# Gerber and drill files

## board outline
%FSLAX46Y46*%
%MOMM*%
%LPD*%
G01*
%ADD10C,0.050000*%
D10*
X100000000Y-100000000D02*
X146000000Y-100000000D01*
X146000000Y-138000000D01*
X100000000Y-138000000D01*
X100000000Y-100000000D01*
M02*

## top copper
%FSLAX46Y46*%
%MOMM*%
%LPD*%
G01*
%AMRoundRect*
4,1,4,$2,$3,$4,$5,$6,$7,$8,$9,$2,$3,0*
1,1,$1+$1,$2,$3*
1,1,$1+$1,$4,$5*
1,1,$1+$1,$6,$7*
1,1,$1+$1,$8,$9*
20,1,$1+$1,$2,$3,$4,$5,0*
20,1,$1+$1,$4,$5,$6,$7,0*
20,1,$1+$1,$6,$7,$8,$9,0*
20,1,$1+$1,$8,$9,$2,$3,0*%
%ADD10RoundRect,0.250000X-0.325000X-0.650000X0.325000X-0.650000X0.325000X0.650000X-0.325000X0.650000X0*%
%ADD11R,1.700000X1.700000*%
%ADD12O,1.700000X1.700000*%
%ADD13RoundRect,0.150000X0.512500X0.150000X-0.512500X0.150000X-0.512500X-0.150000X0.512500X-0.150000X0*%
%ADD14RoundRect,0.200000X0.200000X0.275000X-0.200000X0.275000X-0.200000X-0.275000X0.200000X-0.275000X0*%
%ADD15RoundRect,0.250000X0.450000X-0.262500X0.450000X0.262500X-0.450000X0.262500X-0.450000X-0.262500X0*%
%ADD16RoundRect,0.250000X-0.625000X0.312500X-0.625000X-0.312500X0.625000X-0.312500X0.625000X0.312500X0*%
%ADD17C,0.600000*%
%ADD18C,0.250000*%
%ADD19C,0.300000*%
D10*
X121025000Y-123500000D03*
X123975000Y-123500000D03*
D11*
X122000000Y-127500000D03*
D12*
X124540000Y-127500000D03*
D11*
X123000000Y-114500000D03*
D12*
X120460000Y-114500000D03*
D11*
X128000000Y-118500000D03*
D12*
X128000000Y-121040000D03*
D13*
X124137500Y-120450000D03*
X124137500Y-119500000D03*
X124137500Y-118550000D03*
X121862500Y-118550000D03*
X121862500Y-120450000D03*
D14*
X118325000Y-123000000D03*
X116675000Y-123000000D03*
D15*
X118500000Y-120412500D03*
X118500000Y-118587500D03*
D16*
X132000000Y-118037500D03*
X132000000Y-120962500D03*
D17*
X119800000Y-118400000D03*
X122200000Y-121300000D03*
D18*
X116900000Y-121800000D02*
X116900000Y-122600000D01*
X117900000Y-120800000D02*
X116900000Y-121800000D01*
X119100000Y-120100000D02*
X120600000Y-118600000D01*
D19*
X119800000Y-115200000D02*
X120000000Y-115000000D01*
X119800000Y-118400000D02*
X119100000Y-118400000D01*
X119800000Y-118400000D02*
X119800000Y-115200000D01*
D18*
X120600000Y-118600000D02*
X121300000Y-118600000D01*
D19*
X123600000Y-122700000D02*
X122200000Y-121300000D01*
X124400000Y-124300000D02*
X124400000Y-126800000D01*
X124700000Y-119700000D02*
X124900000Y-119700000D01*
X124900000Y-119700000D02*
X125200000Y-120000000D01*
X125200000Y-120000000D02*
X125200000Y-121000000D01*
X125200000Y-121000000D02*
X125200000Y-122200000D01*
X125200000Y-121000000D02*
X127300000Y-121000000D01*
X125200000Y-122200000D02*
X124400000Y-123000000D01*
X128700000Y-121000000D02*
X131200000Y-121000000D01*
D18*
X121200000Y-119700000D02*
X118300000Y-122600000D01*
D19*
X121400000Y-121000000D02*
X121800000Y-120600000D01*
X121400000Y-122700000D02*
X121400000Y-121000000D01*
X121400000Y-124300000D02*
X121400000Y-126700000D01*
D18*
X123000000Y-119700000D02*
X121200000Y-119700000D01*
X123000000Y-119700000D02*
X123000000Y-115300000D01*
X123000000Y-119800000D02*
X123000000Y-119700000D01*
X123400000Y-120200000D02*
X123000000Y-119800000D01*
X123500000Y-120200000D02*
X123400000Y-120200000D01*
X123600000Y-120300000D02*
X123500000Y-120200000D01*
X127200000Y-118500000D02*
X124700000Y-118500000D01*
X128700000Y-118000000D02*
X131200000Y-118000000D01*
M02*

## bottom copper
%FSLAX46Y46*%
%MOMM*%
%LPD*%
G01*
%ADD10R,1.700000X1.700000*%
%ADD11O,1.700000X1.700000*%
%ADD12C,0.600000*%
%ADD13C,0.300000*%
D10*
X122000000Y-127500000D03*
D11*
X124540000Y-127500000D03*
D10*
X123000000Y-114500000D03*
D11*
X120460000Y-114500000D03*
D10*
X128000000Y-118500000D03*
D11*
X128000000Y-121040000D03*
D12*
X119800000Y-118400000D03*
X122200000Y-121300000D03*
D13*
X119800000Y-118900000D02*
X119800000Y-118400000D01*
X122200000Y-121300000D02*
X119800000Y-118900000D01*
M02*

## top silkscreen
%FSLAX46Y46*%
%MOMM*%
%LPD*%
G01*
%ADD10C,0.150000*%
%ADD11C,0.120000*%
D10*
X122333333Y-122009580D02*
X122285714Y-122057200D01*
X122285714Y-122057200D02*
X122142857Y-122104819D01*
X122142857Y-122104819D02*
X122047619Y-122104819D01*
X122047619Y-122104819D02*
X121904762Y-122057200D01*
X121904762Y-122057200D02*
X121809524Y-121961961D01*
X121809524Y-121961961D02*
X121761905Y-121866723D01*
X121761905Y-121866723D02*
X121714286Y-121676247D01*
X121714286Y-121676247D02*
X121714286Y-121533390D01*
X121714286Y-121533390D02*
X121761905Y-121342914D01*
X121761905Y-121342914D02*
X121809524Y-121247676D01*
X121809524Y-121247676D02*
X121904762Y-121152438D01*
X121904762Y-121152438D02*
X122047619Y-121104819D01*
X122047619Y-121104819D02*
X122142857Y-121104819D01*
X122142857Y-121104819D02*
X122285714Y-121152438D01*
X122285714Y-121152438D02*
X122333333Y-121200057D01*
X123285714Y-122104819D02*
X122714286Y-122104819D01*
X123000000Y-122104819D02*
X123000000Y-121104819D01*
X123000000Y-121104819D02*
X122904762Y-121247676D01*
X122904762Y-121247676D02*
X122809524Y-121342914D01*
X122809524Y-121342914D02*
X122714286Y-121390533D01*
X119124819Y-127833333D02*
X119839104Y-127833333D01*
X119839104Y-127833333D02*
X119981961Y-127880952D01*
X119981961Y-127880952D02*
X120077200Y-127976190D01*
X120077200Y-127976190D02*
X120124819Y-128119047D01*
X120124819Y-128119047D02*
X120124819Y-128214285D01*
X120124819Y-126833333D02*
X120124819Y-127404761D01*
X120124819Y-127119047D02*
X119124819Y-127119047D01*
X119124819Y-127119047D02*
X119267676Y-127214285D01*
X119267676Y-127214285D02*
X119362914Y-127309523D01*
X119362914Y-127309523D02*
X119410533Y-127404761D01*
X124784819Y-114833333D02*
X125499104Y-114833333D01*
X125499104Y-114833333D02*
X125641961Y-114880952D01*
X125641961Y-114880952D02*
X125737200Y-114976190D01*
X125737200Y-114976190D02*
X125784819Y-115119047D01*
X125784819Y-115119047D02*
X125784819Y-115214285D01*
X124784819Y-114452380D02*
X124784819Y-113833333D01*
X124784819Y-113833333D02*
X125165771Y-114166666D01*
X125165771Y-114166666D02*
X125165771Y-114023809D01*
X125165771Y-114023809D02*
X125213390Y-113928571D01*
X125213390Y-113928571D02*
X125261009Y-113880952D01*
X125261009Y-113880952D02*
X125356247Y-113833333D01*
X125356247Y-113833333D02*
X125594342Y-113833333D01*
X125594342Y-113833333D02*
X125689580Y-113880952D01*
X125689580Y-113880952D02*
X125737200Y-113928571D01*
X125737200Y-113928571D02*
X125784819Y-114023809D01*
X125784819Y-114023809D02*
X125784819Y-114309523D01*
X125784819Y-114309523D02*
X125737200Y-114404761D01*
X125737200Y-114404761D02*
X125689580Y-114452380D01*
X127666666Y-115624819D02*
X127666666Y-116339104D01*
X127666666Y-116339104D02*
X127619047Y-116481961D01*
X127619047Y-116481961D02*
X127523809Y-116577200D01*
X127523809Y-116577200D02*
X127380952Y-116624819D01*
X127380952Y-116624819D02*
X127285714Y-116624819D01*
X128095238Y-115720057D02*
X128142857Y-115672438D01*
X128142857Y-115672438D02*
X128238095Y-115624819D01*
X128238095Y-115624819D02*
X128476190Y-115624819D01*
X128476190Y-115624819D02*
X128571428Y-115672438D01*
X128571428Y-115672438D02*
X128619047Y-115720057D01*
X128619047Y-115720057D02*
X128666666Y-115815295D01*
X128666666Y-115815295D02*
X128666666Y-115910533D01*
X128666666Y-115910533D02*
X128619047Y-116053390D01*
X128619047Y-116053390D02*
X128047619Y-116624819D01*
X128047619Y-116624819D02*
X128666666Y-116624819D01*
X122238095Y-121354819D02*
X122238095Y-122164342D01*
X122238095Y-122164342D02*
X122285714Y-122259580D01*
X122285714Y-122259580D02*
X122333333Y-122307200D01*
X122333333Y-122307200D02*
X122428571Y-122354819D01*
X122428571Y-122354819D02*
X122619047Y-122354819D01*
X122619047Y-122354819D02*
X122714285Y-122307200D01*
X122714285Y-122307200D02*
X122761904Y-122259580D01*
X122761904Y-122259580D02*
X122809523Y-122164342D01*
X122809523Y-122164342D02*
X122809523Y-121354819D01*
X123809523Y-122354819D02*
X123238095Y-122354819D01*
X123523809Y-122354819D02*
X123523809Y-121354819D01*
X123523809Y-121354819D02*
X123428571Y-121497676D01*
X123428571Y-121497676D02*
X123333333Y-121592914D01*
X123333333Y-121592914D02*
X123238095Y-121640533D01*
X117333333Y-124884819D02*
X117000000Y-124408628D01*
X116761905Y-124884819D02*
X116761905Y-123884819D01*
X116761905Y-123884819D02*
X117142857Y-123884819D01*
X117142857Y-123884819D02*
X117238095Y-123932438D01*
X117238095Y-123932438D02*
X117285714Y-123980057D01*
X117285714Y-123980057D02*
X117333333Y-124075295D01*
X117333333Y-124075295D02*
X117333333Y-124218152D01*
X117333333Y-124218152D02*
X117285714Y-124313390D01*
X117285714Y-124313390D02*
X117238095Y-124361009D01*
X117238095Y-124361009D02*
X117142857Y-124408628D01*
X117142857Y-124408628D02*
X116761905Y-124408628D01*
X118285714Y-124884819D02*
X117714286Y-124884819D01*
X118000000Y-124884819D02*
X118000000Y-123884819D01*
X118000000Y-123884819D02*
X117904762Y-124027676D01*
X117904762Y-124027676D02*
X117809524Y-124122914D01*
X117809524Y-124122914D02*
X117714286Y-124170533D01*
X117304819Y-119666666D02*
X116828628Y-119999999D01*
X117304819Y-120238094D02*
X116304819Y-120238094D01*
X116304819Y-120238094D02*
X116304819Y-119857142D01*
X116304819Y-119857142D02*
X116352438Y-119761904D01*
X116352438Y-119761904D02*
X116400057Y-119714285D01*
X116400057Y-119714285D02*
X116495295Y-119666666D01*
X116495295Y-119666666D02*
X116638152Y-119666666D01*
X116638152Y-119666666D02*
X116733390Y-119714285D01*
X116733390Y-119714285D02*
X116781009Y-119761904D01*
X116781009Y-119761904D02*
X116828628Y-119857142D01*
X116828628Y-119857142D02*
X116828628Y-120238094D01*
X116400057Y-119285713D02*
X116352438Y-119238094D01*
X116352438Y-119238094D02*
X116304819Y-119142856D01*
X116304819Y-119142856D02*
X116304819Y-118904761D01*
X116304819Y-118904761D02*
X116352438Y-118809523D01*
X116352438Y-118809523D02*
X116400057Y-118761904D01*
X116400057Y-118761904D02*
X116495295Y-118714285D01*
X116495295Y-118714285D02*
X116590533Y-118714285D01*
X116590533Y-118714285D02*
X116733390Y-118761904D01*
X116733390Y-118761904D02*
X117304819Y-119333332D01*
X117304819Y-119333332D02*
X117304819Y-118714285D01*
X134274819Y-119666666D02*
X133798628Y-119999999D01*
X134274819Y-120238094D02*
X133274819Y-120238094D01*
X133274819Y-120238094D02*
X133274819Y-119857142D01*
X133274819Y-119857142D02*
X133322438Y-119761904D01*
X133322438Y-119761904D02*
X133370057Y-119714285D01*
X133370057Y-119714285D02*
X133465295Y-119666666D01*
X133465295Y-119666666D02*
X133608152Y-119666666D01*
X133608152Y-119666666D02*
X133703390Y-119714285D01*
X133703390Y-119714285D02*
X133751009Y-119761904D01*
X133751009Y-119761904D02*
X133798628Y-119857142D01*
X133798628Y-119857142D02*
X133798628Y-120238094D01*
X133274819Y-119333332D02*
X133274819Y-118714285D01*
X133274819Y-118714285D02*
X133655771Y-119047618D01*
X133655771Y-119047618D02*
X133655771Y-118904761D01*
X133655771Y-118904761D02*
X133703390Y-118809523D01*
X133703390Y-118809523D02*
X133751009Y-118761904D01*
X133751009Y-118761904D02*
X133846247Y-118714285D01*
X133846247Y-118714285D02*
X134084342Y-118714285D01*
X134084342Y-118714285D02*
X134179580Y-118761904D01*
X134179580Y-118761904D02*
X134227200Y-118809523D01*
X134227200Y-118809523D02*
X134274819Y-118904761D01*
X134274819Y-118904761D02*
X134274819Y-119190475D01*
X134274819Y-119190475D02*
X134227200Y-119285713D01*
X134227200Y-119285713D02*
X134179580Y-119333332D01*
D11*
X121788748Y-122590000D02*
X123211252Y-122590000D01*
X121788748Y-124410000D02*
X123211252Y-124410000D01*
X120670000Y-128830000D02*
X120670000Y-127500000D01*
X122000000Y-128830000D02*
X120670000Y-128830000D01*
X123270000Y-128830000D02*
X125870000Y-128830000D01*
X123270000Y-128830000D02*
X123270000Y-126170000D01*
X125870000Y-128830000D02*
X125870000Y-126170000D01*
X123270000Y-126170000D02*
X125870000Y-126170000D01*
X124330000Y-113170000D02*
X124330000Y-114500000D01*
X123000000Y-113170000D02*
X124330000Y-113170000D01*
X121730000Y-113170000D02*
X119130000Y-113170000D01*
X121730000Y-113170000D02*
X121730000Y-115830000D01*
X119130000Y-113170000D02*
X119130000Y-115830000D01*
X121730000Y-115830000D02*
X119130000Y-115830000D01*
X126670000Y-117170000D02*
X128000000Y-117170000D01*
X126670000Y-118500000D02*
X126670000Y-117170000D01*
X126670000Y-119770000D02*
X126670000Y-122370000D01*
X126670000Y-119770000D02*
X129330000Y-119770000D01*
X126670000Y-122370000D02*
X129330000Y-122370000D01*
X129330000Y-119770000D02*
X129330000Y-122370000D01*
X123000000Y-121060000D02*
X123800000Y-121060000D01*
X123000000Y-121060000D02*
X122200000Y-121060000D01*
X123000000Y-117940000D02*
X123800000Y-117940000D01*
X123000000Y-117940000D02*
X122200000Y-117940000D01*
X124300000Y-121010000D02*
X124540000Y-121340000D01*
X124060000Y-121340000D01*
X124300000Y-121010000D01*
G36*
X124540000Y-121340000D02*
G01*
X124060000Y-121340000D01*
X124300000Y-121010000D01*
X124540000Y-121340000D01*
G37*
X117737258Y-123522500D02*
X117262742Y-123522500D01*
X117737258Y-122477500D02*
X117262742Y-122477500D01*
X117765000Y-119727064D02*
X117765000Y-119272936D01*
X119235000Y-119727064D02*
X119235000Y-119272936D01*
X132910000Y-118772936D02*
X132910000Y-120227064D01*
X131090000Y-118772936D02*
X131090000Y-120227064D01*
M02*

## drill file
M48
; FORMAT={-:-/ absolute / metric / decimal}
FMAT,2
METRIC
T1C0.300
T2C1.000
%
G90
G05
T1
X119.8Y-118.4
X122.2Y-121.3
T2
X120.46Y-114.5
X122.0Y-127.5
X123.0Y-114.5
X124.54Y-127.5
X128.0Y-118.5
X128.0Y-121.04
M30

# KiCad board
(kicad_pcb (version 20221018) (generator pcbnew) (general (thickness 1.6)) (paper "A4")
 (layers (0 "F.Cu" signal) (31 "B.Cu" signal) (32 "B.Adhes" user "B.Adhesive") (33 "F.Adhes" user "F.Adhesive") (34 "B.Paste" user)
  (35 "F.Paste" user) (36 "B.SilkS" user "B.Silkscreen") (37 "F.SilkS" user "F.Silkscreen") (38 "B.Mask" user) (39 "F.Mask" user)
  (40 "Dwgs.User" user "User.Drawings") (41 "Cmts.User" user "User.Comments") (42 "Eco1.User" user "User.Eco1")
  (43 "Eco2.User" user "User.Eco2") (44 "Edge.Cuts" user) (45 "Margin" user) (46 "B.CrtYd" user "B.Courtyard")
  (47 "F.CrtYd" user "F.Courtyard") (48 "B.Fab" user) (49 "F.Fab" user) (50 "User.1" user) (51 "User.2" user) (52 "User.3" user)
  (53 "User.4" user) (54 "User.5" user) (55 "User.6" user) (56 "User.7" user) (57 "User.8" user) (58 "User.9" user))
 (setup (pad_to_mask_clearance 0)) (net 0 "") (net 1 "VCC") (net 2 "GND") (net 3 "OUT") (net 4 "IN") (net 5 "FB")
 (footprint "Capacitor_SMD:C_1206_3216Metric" (layer "F.Cu") (at 122.5 123.5)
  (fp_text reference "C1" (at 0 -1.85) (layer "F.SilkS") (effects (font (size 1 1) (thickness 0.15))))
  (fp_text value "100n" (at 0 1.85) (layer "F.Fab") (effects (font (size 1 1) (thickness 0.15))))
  (fp_line (start -0.711252 -0.91) (end 0.711252 -0.91) (stroke (width 0.12) (type solid)) (layer "F.SilkS"))
  (fp_line (start -0.711252 0.91) (end 0.711252 0.91) (stroke (width 0.12) (type solid)) (layer "F.SilkS"))
  (pad "1" smd roundrect (at -1.475 0) (size 1.15 1.8) (layers "F.Cu" "F.Paste" "F.Mask") (roundrect_rratio 0.217391) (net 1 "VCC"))
  (pad "2" smd roundrect (at 1.475 0) (size 1.15 1.8) (layers "F.Cu" "F.Paste" "F.Mask") (roundrect_rratio 0.217391) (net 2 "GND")))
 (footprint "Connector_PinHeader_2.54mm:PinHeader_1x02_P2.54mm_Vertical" (layer "F.Cu") (at 122 127.5 90)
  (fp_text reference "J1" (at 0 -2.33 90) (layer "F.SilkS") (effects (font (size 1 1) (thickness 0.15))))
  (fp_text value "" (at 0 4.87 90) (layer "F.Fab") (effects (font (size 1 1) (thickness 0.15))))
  (fp_line (start -1.33 -1.33) (end 0 -1.33) (stroke (width 0.12) (type solid)) (layer "F.SilkS"))
  (fp_line (start -1.33 0) (end -1.33 -1.33) (stroke (width 0.12) (type solid)) (layer "F.SilkS"))
  (fp_line (start -1.33 1.27) (end -1.33 3.87) (stroke (width 0.12) (type solid)) (layer "F.SilkS"))
  (fp_line (start -1.33 1.27) (end 1.33 1.27) (stroke (width 0.12) (type solid)) (layer "F.SilkS"))
  (fp_line (start -1.33 3.87) (end 1.33 3.87) (stroke (width 0.12) (type solid)) (layer "F.SilkS"))
  (fp_line (start 1.33 1.27) (end 1.33 3.87) (stroke (width 0.12) (type solid)) (layer "F.SilkS"))
  (pad "1" thru_hole rect (at 0 0 90) (size 1.7 1.7) (drill 1) (layers "*.Cu" "*.Mask") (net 1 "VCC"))
  (pad "2" thru_hole oval (at 0 2.54 90) (size 1.7 1.7) (drill 1) (layers "*.Cu" "*.Mask") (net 2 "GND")))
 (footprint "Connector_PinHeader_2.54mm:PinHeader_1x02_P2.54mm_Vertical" (layer "F.Cu") (at 123 114.5 -90)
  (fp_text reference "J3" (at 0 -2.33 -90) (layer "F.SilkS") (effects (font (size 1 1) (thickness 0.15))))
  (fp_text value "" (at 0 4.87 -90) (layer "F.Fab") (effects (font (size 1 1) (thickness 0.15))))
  (fp_line (start -1.33 -1.33) (end 0 -1.33) (stroke (width 0.12) (type solid)) (layer "F.SilkS"))
  (fp_line (start -1.33 0) (end -1.33 -1.33) (stroke (width 0.12) (type solid)) (layer "F.SilkS"))
  (fp_line (start -1.33 1.27) (end -1.33 3.87) (stroke (width 0.12) (type solid)) (layer "F.SilkS"))
  (fp_line (start -1.33 1.27) (end 1.33 1.27) (stroke (width 0.12) (type solid)) (layer "F.SilkS"))
  (fp_line (start -1.33 3.87) (end 1.33 3.87) (stroke (width 0.12) (type solid)) (layer "F.SilkS"))
  (fp_line (start 1.33 1.27) (end 1.33 3.87) (stroke (width 0.12) (type solid)) (layer "F.SilkS"))
  (pad "1" thru_hole rect (at 0 0 270) (size 1.7 1.7) (drill 1) (layers "*.Cu" "*.Mask") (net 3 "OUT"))
  (pad "2" thru_hole oval (at 0 2.54 270) (size 1.7 1.7) (drill 1) (layers "*.Cu" "*.Mask") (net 2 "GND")))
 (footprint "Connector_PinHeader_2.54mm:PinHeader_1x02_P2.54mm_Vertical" (layer "F.Cu") (at 128 118.5)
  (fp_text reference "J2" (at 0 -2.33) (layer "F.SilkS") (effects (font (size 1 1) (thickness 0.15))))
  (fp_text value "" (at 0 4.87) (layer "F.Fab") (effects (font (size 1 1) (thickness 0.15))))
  (fp_line (start -1.33 -1.33) (end 0 -1.33) (stroke (width 0.12) (type solid)) (layer "F.SilkS"))
  (fp_line (start -1.33 0) (end -1.33 -1.33) (stroke (width 0.12) (type solid)) (layer "F.SilkS"))
  (fp_line (start -1.33 1.27) (end -1.33 3.87) (stroke (width 0.12) (type solid)) (layer "F.SilkS"))
  (fp_line (start -1.33 1.27) (end 1.33 1.27) (stroke (width 0.12) (type solid)) (layer "F.SilkS"))
  (fp_line (start -1.33 3.87) (end 1.33 3.87) (stroke (width 0.12) (type solid)) (layer "F.SilkS"))
  (fp_line (start 1.33 1.27) (end 1.33 3.87) (stroke (width 0.12) (type solid)) (layer "F.SilkS"))
  (pad "1" thru_hole rect (at 0 0) (size 1.7 1.7) (drill 1) (layers "*.Cu" "*.Mask") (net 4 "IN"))
  (pad "2" thru_hole oval (at 0 2.54) (size 1.7 1.7) (drill 1) (layers "*.Cu" "*.Mask") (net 2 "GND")))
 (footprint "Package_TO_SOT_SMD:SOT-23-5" (layer "F.Cu") (at 123 119.5 180)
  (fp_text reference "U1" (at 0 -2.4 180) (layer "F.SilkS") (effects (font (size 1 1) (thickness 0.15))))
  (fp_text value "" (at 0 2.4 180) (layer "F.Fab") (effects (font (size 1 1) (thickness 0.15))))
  (fp_line (start 0 -1.56) (end -0.8 -1.56) (stroke (width 0.12) (type solid)) (layer "F.SilkS"))
  (fp_line (start 0 -1.56) (end 0.8 -1.56) (stroke (width 0.12) (type solid)) (layer "F.SilkS"))
  (fp_line (start 0 1.56) (end -0.8 1.56) (stroke (width 0.12) (type solid)) (layer "F.SilkS"))
  (fp_line (start 0 1.56) (end 0.8 1.56) (stroke (width 0.12) (type solid)) (layer "F.SilkS"))
  (fp_poly
   (pts (xy -1.3 -1.51) (xy -1.54 -1.84) (xy -1.06 -1.84) (xy -1.3 -1.51)) (stroke (width 0.12) (type solid)) (fill solid) (layer "F.SilkS"))
  (pad "1" smd roundrect (at -1.1375 -0.95 180) (size 1.325 0.6) (layers "F.Cu" "F.Paste" "F.Mask") (roundrect_rratio 0.25) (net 3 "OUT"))
  (pad "2" smd roundrect (at -1.1375 0 180) (size 1.325 0.6) (layers "F.Cu" "F.Paste" "F.Mask") (roundrect_rratio 0.25) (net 2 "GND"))
  (pad "3" smd roundrect (at -1.1375 0.95 180) (size 1.325 0.6) (layers "F.Cu" "F.Paste" "F.Mask") (roundrect_rratio 0.25) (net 4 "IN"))
  (pad "4" smd roundrect (at 1.1375 0.95 180) (size 1.325 0.6) (layers "F.Cu" "F.Paste" "F.Mask") (roundrect_rratio 0.25) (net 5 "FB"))
  (pad "5" smd roundrect (at 1.1375 -0.95 180) (size 1.325 0.6) (layers "F.Cu" "F.Paste" "F.Mask") (roundrect_rratio 0.25) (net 1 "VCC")))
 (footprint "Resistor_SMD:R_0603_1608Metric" (layer "F.Cu") (at 117.5 123 180)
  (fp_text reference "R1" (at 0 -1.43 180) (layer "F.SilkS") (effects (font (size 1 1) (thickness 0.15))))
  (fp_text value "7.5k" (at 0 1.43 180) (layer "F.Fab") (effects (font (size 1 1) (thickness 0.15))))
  (fp_line (start -0.237258 -0.5225) (end 0.237258 -0.5225) (stroke (width 0.12) (type solid)) (layer "F.SilkS"))
  (fp_line (start -0.237258 0.5225) (end 0.237258 0.5225) (stroke (width 0.12) (type solid)) (layer "F.SilkS"))
  (pad "1" smd roundrect (at -0.825 0 180) (size 0.8 0.95) (layers "F.Cu" "F.Paste" "F.Mask") (roundrect_rratio 0.25) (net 3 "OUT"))
  (pad "2" smd roundrect (at 0.825 0 180) (size 0.8 0.95) (layers "F.Cu" "F.Paste" "F.Mask") (roundrect_rratio 0.25) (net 5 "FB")))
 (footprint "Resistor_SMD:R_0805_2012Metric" (layer "F.Cu") (at 118.5 119.5 90)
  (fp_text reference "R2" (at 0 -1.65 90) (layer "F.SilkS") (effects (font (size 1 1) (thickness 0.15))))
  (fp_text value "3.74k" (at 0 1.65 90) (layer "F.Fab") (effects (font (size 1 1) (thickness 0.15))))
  (fp_line (start -0.227064 -0.735) (end 0.227064 -0.735) (stroke (width 0.12) (type solid)) (layer "F.SilkS"))
  (fp_line (start -0.227064 0.735) (end 0.227064 0.735) (stroke (width 0.12) (type solid)) (layer "F.SilkS"))
  (pad "1" smd roundrect (at -0.9125 0 90) (size 1.025 1.4) (layers "F.Cu" "F.Paste" "F.Mask") (roundrect_rratio 0.243902) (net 5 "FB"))
  (pad "2" smd roundrect (at 0.9125 0 90) (size 1.025 1.4) (layers "F.Cu" "F.Paste" "F.Mask") (roundrect_rratio 0.243902) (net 2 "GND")))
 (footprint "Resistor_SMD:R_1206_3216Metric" (layer "F.Cu") (at 132 119.5 -90)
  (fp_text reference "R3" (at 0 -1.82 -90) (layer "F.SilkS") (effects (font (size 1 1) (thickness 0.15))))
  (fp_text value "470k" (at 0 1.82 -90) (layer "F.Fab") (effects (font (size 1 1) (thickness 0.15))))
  (fp_line (start -0.727064 -0.91) (end 0.727064 -0.91) (stroke (width 0.12) (type solid)) (layer "F.SilkS"))
  (fp_line (start -0.727064 0.91) (end 0.727064 0.91) (stroke (width 0.12) (type solid)) (layer "F.SilkS"))
  (pad "1" smd roundrect (at -1.4625 0 270) (size 1.125 1.75) (layers "F.Cu" "F.Paste" "F.Mask") (roundrect_rratio 0.222222) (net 4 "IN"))
  (pad "2" smd roundrect (at 1.4625 0 270) (size 1.125 1.75) (layers "F.Cu" "F.Paste" "F.Mask") (roundrect_rratio 0.222222) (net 2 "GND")))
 (gr_rect (start 100 100) (end 146 138) (stroke (width 0.05) (type default)) (fill none) (layer "Edge.Cuts"))
 (segment (start 116.9 121.8) (end 116.9 122.6) (width 0.25) (layer "F.Cu") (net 5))
 (segment (start 117.9 120.8) (end 116.9 121.8) (width 0.25) (layer "F.Cu") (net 5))
 (segment (start 119.1 120.1) (end 120.6 118.6) (width 0.25) (layer "F.Cu") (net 5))
 (segment (start 119.8 115.2) (end 120 115) (width 0.3) (layer "F.Cu") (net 2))
 (segment (start 119.8 118.4) (end 119.1 118.4) (width 0.3) (layer "F.Cu") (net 2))
 (segment (start 119.8 118.4) (end 119.8 115.2) (width 0.3) (layer "F.Cu") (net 2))
 (segment (start 120.6 118.6) (end 121.3 118.6) (width 0.25) (layer "F.Cu") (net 5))
 (segment (start 123.6 122.7) (end 122.2 121.3) (width 0.3) (layer "F.Cu") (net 2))
 (segment (start 124.4 124.3) (end 124.4 126.8) (width 0.3) (layer "F.Cu") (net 2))
 (segment (start 124.7 119.7) (end 124.9 119.7) (width 0.3) (layer "F.Cu") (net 2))
 (segment (start 124.9 119.7) (end 125.2 120) (width 0.3) (layer "F.Cu") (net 2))
 (segment (start 125.2 120) (end 125.2 121) (width 0.3) (layer "F.Cu") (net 2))
 (segment (start 125.2 121) (end 125.2 122.2) (width 0.3) (layer "F.Cu") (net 2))
 (segment (start 125.2 121) (end 127.3 121) (width 0.3) (layer "F.Cu") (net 2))
 (segment (start 125.2 122.2) (end 124.4 123) (width 0.3) (layer "F.Cu") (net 2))
 (segment (start 128.7 121) (end 131.2 121) (width 0.3) (layer "F.Cu") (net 2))
 (via (at 119.8 118.4) (size 0.6) (drill 0.3) (layers "F.Cu" "B.Cu") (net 2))
 (via (at 122.2 121.3) (size 0.6) (drill 0.3) (layers "F.Cu" "B.Cu") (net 2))
 (segment (start 119.8 118.9) (end 119.8 118.4) (width 0.3) (layer "B.Cu") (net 2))
 (segment (start 121.2 119.7) (end 118.3 122.6) (width 0.25) (layer "F.Cu") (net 3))
 (segment (start 121.4 121) (end 121.8 120.6) (width 0.3) (layer "F.Cu") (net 1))
 (segment (start 121.4 122.7) (end 121.4 121) (width 0.3) (layer "F.Cu") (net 1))
 (segment (start 121.4 124.3) (end 121.4 126.7) (width 0.3) (layer "F.Cu") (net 1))
 (segment (start 122.2 121.3) (end 119.8 118.9) (width 0.3) (layer "B.Cu") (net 2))
 (segment (start 123 119.7) (end 121.2 119.7) (width 0.25) (layer "F.Cu") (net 3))
 (segment (start 123 119.7) (end 123 115.3) (width 0.25) (layer "F.Cu") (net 3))
 (segment (start 123 119.8) (end 123 119.7) (width 0.25) (layer "F.Cu") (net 3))
 (segment (start 123.4 120.2) (end 123 119.8) (width 0.25) (layer "F.Cu") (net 3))
 (segment (start 123.5 120.2) (end 123.4 120.2) (width 0.25) (layer "F.Cu") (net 3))
 (segment (start 123.6 120.3) (end 123.5 120.2) (width 0.25) (layer "F.Cu") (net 3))
 (segment (start 127.2 118.5) (end 124.7 118.5) (width 0.25) (layer "F.Cu") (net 4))
 (segment (start 128.7 118) (end 131.2 118) (width 0.25) (layer "F.Cu") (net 4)))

